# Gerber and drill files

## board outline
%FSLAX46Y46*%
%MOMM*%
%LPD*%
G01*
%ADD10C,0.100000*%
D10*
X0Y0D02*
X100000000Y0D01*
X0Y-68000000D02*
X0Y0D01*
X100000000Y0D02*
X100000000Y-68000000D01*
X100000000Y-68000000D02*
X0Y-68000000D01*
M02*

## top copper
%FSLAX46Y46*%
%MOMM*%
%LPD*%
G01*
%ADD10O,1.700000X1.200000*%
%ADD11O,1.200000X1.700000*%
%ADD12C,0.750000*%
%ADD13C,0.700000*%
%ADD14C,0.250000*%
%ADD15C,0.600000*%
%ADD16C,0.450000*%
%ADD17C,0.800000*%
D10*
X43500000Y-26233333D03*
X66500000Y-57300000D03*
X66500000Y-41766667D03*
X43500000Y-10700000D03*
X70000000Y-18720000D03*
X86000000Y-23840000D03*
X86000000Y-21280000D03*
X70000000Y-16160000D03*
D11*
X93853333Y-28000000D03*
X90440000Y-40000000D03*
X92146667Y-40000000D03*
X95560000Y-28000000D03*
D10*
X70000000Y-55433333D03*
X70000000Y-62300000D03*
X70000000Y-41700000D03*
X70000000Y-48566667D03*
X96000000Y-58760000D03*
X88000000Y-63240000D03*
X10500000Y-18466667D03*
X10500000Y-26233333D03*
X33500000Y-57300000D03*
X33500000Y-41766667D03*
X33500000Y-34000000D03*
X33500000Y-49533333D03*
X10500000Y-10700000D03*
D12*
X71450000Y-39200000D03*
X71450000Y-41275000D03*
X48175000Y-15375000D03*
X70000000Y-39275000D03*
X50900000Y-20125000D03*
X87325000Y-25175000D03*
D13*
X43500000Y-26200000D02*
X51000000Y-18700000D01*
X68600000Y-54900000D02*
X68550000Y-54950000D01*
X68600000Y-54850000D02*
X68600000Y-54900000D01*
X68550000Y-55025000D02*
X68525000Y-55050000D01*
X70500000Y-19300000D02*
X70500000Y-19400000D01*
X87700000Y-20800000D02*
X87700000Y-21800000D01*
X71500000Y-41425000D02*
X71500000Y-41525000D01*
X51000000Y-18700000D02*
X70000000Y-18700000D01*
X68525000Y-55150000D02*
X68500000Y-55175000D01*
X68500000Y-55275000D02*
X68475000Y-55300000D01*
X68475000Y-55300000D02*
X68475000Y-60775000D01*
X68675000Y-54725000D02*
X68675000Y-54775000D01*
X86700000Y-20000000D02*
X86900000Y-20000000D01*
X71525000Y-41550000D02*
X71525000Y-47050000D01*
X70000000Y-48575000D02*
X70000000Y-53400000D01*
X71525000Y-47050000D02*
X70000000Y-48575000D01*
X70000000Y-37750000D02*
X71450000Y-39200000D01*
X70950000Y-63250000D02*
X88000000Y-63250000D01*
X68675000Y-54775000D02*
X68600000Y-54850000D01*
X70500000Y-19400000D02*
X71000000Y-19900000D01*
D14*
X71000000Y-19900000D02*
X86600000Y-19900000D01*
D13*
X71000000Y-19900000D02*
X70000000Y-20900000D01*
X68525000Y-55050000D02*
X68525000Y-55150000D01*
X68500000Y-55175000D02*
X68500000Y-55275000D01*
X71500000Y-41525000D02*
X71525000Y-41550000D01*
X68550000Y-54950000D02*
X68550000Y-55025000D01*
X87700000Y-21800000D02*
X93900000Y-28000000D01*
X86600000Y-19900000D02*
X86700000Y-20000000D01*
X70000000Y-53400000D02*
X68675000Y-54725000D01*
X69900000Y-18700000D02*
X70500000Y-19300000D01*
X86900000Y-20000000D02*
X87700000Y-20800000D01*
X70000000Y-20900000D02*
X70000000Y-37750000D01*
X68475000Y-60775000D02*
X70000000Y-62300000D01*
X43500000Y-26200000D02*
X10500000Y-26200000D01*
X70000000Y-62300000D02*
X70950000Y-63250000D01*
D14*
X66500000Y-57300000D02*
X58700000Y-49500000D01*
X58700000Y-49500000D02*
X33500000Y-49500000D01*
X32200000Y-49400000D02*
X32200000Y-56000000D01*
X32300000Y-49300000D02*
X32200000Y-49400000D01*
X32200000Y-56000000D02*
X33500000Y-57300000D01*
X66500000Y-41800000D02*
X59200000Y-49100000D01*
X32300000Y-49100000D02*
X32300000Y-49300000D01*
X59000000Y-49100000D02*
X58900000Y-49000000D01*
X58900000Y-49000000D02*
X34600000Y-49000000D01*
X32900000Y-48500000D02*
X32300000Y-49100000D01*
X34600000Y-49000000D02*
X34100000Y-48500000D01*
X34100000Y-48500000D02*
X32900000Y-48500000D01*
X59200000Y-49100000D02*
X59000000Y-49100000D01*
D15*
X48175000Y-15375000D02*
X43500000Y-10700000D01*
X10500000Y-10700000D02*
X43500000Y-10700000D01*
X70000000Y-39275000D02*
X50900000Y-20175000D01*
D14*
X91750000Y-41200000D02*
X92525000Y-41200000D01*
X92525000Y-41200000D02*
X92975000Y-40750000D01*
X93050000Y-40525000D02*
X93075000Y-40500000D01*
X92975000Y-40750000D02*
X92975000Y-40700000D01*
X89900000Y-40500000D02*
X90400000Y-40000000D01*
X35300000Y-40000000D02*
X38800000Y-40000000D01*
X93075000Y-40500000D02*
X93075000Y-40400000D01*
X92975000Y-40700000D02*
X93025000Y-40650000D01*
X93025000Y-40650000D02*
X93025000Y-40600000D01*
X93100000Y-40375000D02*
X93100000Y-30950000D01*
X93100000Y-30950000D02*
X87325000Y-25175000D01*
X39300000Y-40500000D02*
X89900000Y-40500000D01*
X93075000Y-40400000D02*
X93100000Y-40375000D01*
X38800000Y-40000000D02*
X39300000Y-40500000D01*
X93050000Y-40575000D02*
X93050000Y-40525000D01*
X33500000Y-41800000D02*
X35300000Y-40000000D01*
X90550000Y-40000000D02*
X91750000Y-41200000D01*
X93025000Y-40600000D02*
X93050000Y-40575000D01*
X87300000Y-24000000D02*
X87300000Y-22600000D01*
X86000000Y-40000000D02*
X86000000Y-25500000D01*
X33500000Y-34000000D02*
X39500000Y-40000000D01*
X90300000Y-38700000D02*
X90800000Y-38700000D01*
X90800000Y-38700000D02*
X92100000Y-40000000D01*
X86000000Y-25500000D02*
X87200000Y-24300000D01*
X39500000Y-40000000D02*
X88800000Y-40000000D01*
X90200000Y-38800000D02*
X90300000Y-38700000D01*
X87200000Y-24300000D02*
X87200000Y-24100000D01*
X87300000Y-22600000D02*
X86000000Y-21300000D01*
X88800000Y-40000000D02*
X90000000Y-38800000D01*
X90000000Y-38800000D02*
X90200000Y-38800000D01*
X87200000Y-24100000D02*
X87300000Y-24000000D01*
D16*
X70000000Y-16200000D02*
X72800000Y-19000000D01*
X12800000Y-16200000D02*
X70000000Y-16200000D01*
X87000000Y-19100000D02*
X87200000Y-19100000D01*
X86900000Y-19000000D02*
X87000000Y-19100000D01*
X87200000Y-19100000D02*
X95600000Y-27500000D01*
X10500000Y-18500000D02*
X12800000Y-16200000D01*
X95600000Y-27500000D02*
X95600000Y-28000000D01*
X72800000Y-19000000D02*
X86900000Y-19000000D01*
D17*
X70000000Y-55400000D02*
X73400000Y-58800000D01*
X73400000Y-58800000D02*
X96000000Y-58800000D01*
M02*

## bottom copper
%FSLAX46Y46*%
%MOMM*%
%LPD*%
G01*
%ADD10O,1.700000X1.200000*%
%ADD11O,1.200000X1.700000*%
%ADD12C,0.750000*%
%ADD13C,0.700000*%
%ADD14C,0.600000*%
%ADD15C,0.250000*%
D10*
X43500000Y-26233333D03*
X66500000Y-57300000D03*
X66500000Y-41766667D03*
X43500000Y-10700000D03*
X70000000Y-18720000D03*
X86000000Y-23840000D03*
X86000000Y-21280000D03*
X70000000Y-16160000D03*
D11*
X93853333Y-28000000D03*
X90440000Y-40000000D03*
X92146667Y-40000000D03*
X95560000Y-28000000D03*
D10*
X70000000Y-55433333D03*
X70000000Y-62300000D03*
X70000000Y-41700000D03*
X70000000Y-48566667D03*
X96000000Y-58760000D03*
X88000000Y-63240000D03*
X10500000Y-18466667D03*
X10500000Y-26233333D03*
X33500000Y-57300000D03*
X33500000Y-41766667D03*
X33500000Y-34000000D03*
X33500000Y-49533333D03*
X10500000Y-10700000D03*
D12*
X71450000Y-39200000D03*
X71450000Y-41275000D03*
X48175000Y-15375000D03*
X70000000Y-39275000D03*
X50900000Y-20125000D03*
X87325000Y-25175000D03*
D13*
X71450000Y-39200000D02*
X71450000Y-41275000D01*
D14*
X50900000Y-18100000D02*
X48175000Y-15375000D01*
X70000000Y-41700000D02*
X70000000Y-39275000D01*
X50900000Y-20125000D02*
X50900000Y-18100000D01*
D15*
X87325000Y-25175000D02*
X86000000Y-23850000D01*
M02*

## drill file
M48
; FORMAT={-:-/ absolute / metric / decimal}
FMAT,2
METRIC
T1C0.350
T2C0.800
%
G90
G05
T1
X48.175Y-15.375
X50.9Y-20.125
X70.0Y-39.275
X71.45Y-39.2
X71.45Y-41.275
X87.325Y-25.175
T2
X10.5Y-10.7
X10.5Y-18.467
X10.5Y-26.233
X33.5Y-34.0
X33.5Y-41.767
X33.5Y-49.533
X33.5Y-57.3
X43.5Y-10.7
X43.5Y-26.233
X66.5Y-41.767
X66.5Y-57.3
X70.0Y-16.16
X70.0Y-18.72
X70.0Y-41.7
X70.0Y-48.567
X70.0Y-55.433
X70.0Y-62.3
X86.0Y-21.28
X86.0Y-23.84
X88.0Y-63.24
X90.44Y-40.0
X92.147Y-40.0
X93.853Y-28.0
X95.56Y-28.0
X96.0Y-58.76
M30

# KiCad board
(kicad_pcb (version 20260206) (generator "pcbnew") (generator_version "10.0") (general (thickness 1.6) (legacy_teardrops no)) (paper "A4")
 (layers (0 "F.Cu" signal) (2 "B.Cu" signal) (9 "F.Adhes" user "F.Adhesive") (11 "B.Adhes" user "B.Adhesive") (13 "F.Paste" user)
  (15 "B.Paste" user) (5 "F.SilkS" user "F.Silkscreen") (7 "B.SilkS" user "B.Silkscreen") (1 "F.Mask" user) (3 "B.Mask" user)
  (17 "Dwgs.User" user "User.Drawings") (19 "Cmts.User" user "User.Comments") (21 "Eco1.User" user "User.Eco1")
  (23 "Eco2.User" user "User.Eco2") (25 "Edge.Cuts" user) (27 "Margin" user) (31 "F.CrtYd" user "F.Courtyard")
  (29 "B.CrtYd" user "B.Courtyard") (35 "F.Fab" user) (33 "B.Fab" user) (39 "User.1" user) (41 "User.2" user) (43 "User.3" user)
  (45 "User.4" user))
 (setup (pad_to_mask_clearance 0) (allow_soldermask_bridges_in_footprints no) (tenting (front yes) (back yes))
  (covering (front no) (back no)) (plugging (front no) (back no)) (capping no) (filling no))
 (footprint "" (layer "F.Cu") (at 55 34)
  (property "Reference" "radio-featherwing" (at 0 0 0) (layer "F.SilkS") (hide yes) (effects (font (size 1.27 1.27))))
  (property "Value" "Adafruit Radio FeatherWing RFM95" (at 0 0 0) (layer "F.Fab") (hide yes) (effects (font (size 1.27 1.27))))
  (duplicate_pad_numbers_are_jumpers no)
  (pad "GND" thru_hole oval (at -11.5 -7.766667) (size 1.7 1.2) (drill 0.8) (layers "*.Cu") (remove_unused_layers no) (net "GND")
   (thermal_bridge_angle 45))
  (pad "RX" thru_hole oval (at 11.5 23.3) (size 1.7 1.2) (drill 0.8) (layers "*.Cu") (remove_unused_layers no) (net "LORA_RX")
   (thermal_bridge_angle 45))
  (pad "TX" thru_hole oval (at 11.5 7.766667) (size 1.7 1.2) (drill 0.8) (layers "*.Cu") (remove_unused_layers no) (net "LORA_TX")
   (thermal_bridge_angle 45))
  (pad "VCC" thru_hole oval (at -11.5 -23.3) (size 1.7 1.2) (drill 0.8) (layers "*.Cu") (remove_unused_layers no) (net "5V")
   (thermal_bridge_angle 45)))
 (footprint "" (layer "F.Cu") (at 78 20)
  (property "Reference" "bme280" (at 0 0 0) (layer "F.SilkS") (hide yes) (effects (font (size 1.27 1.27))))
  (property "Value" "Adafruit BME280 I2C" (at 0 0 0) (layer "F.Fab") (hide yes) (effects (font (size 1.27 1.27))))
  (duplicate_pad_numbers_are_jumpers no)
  (pad "GND" thru_hole oval (at -8 -1.28) (size 1.7 1.2) (drill 0.8) (layers "*.Cu") (remove_unused_layers no) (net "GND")
   (thermal_bridge_angle 45))
  (pad "SCL" thru_hole oval (at 8 3.84) (size 1.7 1.2) (drill 0.8) (layers "*.Cu") (remove_unused_layers no) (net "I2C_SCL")
   (thermal_bridge_angle 45))
  (pad "SDA" thru_hole oval (at 8 1.28) (size 1.7 1.2) (drill 0.8) (layers "*.Cu") (remove_unused_layers no) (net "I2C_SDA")
   (thermal_bridge_angle 45))
  (pad "VCC" thru_hole oval (at -8 -3.84) (size 1.7 1.2) (drill 0.8) (layers "*.Cu") (remove_unused_layers no) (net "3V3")
   (thermal_bridge_angle 45)))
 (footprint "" (layer "F.Cu") (at 93 34 90)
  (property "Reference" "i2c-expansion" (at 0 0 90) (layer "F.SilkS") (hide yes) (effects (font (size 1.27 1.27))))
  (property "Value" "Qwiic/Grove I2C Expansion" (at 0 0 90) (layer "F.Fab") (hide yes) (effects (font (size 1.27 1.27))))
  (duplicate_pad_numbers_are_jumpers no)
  (pad "GND" thru_hole oval (at 6 0.853333 90) (size 1.7 1.2) (drill 0.8) (layers "*.Cu") (remove_unused_layers no) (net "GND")
   (thermal_bridge_angle 45))
  (pad "SCL" thru_hole oval (at -6 -2.56 90) (size 1.7 1.2) (drill 0.8) (layers "*.Cu") (remove_unused_layers no) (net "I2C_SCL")
   (thermal_bridge_angle 45))
  (pad "SDA" thru_hole oval (at -6 -0.853333 90) (size 1.7 1.2) (drill 0.8) (layers "*.Cu") (remove_unused_layers no) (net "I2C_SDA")
   (thermal_bridge_angle 45))
  (pad "VCC" thru_hole oval (at 6 2.56 90) (size 1.7 1.2) (drill 0.8) (layers "*.Cu") (remove_unused_layers no) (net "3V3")
   (thermal_bridge_angle 45)))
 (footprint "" (layer "F.Cu") (at 78 52)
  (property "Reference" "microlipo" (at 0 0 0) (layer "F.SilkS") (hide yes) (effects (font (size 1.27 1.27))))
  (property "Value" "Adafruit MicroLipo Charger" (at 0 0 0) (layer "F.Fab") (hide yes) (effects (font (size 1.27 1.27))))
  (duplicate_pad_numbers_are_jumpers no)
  (pad "B+" thru_hole oval (at -8 3.433333) (size 1.7 1.2) (drill 0.8) (layers "*.Cu") (remove_unused_layers no) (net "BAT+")
   (thermal_bridge_angle 45))
  (pad "B-" thru_hole oval (at -8 10.3) (size 1.7 1.2) (drill 0.8) (layers "*.Cu") (remove_unused_layers no) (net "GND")
   (thermal_bridge_angle 45))
  (pad "OUT+" thru_hole oval (at -8 -10.3) (size 1.7 1.2) (drill 0.8) (layers "*.Cu") (remove_unused_layers no) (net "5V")
   (thermal_bridge_angle 45))
  (pad "OUT-" thru_hole oval (at -8 -3.433333) (size 1.7 1.2) (drill 0.8) (layers "*.Cu") (remove_unused_layers no) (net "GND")
   (thermal_bridge_angle 45)))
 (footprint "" (layer "F.Cu") (at 92 61)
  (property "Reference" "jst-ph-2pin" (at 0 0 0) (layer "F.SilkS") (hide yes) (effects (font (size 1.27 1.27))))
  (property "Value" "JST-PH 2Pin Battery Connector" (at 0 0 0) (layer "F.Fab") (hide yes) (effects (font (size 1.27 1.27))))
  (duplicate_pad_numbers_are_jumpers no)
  (pad "BAT+" thru_hole oval (at 4 -2.24) (size 1.7 1.2) (drill 0.8) (layers "*.Cu") (remove_unused_layers no) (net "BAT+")
   (thermal_bridge_angle 45))
  (pad "GND" thru_hole oval (at -4 2.24) (size 1.7 1.2) (drill 0.8) (layers "*.Cu") (remove_unused_layers no) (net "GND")
   (thermal_bridge_angle 45)))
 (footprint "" (layer "F.Cu") (at 22 34)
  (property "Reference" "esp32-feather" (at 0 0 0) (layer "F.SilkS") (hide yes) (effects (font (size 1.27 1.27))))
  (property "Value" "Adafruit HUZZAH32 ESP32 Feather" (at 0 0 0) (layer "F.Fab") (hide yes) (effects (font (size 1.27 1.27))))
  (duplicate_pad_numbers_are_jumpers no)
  (pad "3V3" thru_hole oval (at -11.5 -15.533333) (size 1.7 1.2) (drill 0.8) (layers "*.Cu") (remove_unused_layers no) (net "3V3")
   (thermal_bridge_angle 45))
  (pad "GND" thru_hole oval (at -11.5 -7.766667) (size 1.7 1.2) (drill 0.8) (layers "*.Cu") (remove_unused_layers no) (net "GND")
   (thermal_bridge_angle 45))
  (pad "RX" thru_hole oval (at 11.5 23.3) (size 1.7 1.2) (drill 0.8) (layers "*.Cu") (remove_unused_layers no) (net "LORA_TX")
   (thermal_bridge_angle 45))
  (pad "SCL" thru_hole oval (at 11.5 7.766667) (size 1.7 1.2) (drill 0.8) (layers "*.Cu") (remove_unused_layers no) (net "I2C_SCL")
   (thermal_bridge_angle 45))
  (pad "SDA" thru_hole oval (at 11.5 0) (size 1.7 1.2) (drill 0.8) (layers "*.Cu") (remove_unused_layers no) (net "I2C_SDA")
   (thermal_bridge_angle 45))
  (pad "TX" thru_hole oval (at 11.5 15.533333) (size 1.7 1.2) (drill 0.8) (layers "*.Cu") (remove_unused_layers no) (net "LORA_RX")
   (thermal_bridge_angle 45))
  (pad "VIN" thru_hole oval (at -11.5 -23.3) (size 1.7 1.2) (drill 0.8) (layers "*.Cu") (remove_unused_layers no) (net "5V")
   (thermal_bridge_angle 45)))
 (gr_line (start 0 0) (end 100 0) (stroke (width 0.1) (type default)) (layer "Edge.Cuts"))
 (gr_line (start 0 68) (end 0 0) (stroke (width 0.1) (type default)) (layer "Edge.Cuts"))
 (gr_line (start 100 0) (end 100 68) (stroke (width 0.1) (type default)) (layer "Edge.Cuts"))
 (gr_line (start 100 68) (end 0 68) (stroke (width 0.1) (type default)) (layer "Edge.Cuts"))
 (segment (start 43.5 26.2) (end 51 18.7) (width 0.7) (layer "F.Cu") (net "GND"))
 (segment (start 68.6 54.9) (end 68.55 54.95) (width 0.7) (layer "F.Cu") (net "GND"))
 (segment (start 68.6 54.85) (end 68.6 54.9) (width 0.7) (layer "F.Cu") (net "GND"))
 (segment (start 68.55 55.025) (end 68.525 55.05) (width 0.7) (layer "F.Cu") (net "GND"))
 (segment (start 70.5 19.3) (end 70.5 19.4) (width 0.7) (layer "F.Cu") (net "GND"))
 (segment (start 87.7 20.8) (end 87.7 21.8) (width 0.7) (layer "F.Cu") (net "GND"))
 (segment (start 71.5 41.425) (end 71.5 41.525) (width 0.7) (layer "F.Cu") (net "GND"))
 (segment (start 51 18.7) (end 70 18.7) (width 0.7) (layer "F.Cu") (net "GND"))
 (segment (start 68.525 55.15) (end 68.5 55.175) (width 0.7) (layer "F.Cu") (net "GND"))
 (segment (start 68.5 55.275) (end 68.475 55.3) (width 0.7) (layer "F.Cu") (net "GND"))
 (segment (start 68.475 55.3) (end 68.475 60.775) (width 0.7) (layer "F.Cu") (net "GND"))
 (segment (start 68.675 54.725) (end 68.675 54.775) (width 0.7) (layer "F.Cu") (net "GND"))
 (segment (start 86.7 20) (end 86.9 20) (width 0.7) (layer "F.Cu") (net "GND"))
 (segment (start 71.525 41.55) (end 71.525 47.05) (width 0.7) (layer "F.Cu") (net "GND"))
 (segment (start 70 48.575) (end 70 53.4) (width 0.7) (layer "F.Cu") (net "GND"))
 (segment (start 71.525 47.05) (end 70 48.575) (width 0.7) (layer "F.Cu") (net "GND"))
 (segment (start 70 37.75) (end 71.45 39.2) (width 0.7) (layer "F.Cu") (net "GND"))
 (segment (start 70.95 63.25) (end 88 63.25) (width 0.7) (layer "F.Cu") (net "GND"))
 (segment (start 68.675 54.775) (end 68.6 54.85) (width 0.7) (layer "F.Cu") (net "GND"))
 (segment (start 70.5 19.4) (end 71 19.9) (width 0.7) (layer "F.Cu") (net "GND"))
 (segment (start 71 19.9) (end 86.6 19.9) (width 0.25) (layer "F.Cu") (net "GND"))
 (segment (start 71 19.9) (end 70 20.9) (width 0.7) (layer "F.Cu") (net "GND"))
 (segment (start 68.525 55.05) (end 68.525 55.15) (width 0.7) (layer "F.Cu") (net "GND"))
 (segment (start 68.5 55.175) (end 68.5 55.275) (width 0.7) (layer "F.Cu") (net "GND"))
 (segment (start 71.5 41.525) (end 71.525 41.55) (width 0.7) (layer "F.Cu") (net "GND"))
 (segment (start 68.55 54.95) (end 68.55 55.025) (width 0.7) (layer "F.Cu") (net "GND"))
 (segment (start 87.7 21.8) (end 93.9 28) (width 0.7) (layer "F.Cu") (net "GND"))
 (segment (start 86.6 19.9) (end 86.7 20) (width 0.7) (layer "F.Cu") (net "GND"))
 (segment (start 70 53.4) (end 68.675 54.725) (width 0.7) (layer "F.Cu") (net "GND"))
 (segment (start 69.9 18.7) (end 70.5 19.3) (width 0.7) (layer "F.Cu") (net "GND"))
 (segment (start 86.9 20) (end 87.7 20.8) (width 0.7) (layer "F.Cu") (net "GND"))
 (segment (start 70 20.9) (end 70 37.75) (width 0.7) (layer "F.Cu") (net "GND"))
 (segment (start 68.475 60.775) (end 70 62.3) (width 0.7) (layer "F.Cu") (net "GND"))
 (segment (start 43.5 26.2) (end 10.5 26.2) (width 0.7) (layer "F.Cu") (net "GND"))
 (segment (start 70 62.3) (end 70.95 63.25) (width 0.7) (layer "F.Cu") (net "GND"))
 (via (at 71.45 39.2) (size 0.75) (drill 0.35) (layers "F.Cu" "B.Cu") (tenting (front yes) (back yes)) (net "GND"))
 (via (at 71.45 41.275) (size 0.75) (drill 0.35) (layers "F.Cu" "B.Cu") (tenting (front yes) (back yes)) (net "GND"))
 (segment (start 71.45 39.2) (end 71.45 41.275) (width 0.7) (layer "B.Cu") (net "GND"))
 (segment (start 66.5 57.3) (end 58.7 49.5) (width 0.25) (layer "F.Cu") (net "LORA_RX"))
 (segment (start 58.7 49.5) (end 33.5 49.5) (width 0.25) (layer "F.Cu") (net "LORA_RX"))
 (segment (start 32.2 49.4) (end 32.2 56) (width 0.25) (layer "F.Cu") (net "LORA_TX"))
 (segment (start 32.3 49.3) (end 32.2 49.4) (width 0.25) (layer "F.Cu") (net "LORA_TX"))
 (segment (start 32.2 56) (end 33.5 57.3) (width 0.25) (layer "F.Cu") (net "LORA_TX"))
 (segment (start 66.5 41.8) (end 59.2 49.1) (width 0.25) (layer "F.Cu") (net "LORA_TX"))
 (segment (start 32.3 49.1) (end 32.3 49.3) (width 0.25) (layer "F.Cu") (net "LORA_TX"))
 (segment (start 59 49.1) (end 58.9 49) (width 0.25) (layer "F.Cu") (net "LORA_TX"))
 (segment (start 58.9 49) (end 34.6 49) (width 0.25) (layer "F.Cu") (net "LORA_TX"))
 (segment (start 32.9 48.5) (end 32.3 49.1) (width 0.25) (layer "F.Cu") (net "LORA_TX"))
 (segment (start 34.6 49) (end 34.1 48.5) (width 0.25) (layer "F.Cu") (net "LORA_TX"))
 (segment (start 34.1 48.5) (end 32.9 48.5) (width 0.25) (layer "F.Cu") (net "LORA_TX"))
 (segment (start 59.2 49.1) (end 59 49.1) (width 0.25) (layer "F.Cu") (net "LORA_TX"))
 (segment (start 48.175 15.375) (end 43.5 10.7) (width 0.6) (layer "F.Cu") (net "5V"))
 (segment (start 10.5 10.7) (end 43.5 10.7) (width 0.6) (layer "F.Cu") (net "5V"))
 (segment (start 70 39.275) (end 50.9 20.175) (width 0.6) (layer "F.Cu") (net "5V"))
 (via (at 48.175 15.375) (size 0.75) (drill 0.35) (layers "F.Cu" "B.Cu") (tenting (front yes) (back yes)) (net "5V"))
 (via (at 70 39.275) (size 0.75) (drill 0.35) (layers "F.Cu" "B.Cu") (tenting (front yes) (back yes)) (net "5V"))
 (via (at 50.9 20.125) (size 0.75) (drill 0.35) (layers "F.Cu" "B.Cu") (tenting (front yes) (back yes)) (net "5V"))
 (segment (start 50.9 18.1) (end 48.175 15.375) (width 0.6) (layer "B.Cu") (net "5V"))
 (segment (start 70 41.7) (end 70 39.275) (width 0.6) (layer "B.Cu") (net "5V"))
 (segment (start 50.9 20.125) (end 50.9 18.1) (width 0.6) (layer "B.Cu") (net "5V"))
 (segment (start 91.75 41.2) (end 92.525 41.2) (width 0.25) (layer "F.Cu") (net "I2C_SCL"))
 (segment (start 92.525 41.2) (end 92.975 40.75) (width 0.25) (layer "F.Cu") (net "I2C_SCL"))
 (segment (start 93.05 40.525) (end 93.075 40.5) (width 0.25) (layer "F.Cu") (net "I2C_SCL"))
 (segment (start 92.975 40.75) (end 92.975 40.7) (width 0.25) (layer "F.Cu") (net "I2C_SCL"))
 (segment (start 89.9 40.5) (end 90.4 40) (width 0.25) (layer "F.Cu") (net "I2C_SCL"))
 (segment (start 35.3 40) (end 38.8 40) (width 0.25) (layer "F.Cu") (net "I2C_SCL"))
 (segment (start 93.075 40.5) (end 93.075 40.4) (width 0.25) (layer "F.Cu") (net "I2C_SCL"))
 (segment (start 92.975 40.7) (end 93.025 40.65) (width 0.25) (layer "F.Cu") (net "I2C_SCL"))
 (segment (start 93.025 40.65) (end 93.025 40.6) (width 0.25) (layer "F.Cu") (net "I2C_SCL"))
 (segment (start 93.1 40.375) (end 93.1 30.95) (width 0.25) (layer "F.Cu") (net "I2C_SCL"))
 (segment (start 93.1 30.95) (end 87.325 25.175) (width 0.25) (layer "F.Cu") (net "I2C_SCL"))
 (segment (start 39.3 40.5) (end 89.9 40.5) (width 0.25) (layer "F.Cu") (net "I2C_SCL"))
 (segment (start 93.075 40.4) (end 93.1 40.375) (width 0.25) (layer "F.Cu") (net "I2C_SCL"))
 (segment (start 38.8 40) (end 39.3 40.5) (width 0.25) (layer "F.Cu") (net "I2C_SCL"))
 (segment (start 93.05 40.575) (end 93.05 40.525) (width 0.25) (layer "F.Cu") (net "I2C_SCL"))
 (segment (start 33.5 41.8) (end 35.3 40) (width 0.25) (layer "F.Cu") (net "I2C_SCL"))
 (segment (start 90.55 40) (end 91.75 41.2) (width 0.25) (layer "F.Cu") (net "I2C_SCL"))
 (segment (start 93.025 40.6) (end 93.05 40.575) (width 0.25) (layer "F.Cu") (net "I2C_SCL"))
 (via (at 87.325 25.175) (size 0.75) (drill 0.35) (layers "F.Cu" "B.Cu") (tenting (front yes) (back yes)) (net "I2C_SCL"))
 (segment (start 87.325 25.175) (end 86 23.85) (width 0.25) (layer "B.Cu") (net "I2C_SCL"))
 (segment (start 87.3 24) (end 87.3 22.6) (width 0.25) (layer "F.Cu") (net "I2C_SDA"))
 (segment (start 86 40) (end 86 25.5) (width 0.25) (layer "F.Cu") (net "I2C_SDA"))
 (segment (start 33.5 34) (end 39.5 40) (width 0.25) (layer "F.Cu") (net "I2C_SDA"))
 (segment (start 90.3 38.7) (end 90.8 38.7) (width 0.25) (layer "F.Cu") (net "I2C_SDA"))
 (segment (start 90.8 38.7) (end 92.1 40) (width 0.25) (layer "F.Cu") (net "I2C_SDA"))
 (segment (start 86 25.5) (end 87.2 24.3) (width 0.25) (layer "F.Cu") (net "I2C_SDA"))
 (segment (start 39.5 40) (end 88.8 40) (width 0.25) (layer "F.Cu") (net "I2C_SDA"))
 (segment (start 90.2 38.8) (end 90.3 38.7) (width 0.25) (layer "F.Cu") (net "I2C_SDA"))
 (segment (start 87.2 24.3) (end 87.2 24.1) (width 0.25) (layer "F.Cu") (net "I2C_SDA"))
 (segment (start 87.3 22.6) (end 86 21.3) (width 0.25) (layer "F.Cu") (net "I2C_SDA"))
 (segment (start 88.8 40) (end 90 38.8) (width 0.25) (layer "F.Cu") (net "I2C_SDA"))
 (segment (start 90 38.8) (end 90.2 38.8) (width 0.25) (layer "F.Cu") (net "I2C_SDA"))
 (segment (start 87.2 24.1) (end 87.3 24) (width 0.25) (layer "F.Cu") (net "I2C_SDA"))
 (segment (start 70 16.2) (end 72.8 19) (width 0.45) (layer "F.Cu") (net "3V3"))
 (segment (start 12.8 16.2) (end 70 16.2) (width 0.45) (layer "F.Cu") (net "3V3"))
 (segment (start 87 19.1) (end 87.2 19.1) (width 0.45) (layer "F.Cu") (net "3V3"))
 (segment (start 86.9 19) (end 87 19.1) (width 0.45) (layer "F.Cu") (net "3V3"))
 (segment (start 87.2 19.1) (end 95.6 27.5) (width 0.45) (layer "F.Cu") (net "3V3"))
 (segment (start 10.5 18.5) (end 12.8 16.2) (width 0.45) (layer "F.Cu") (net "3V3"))
 (segment (start 95.6 27.5) (end 95.6 28) (width 0.45) (layer "F.Cu") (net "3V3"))
 (segment (start 72.8 19) (end 86.9 19) (width 0.45) (layer "F.Cu") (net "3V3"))
 (segment (start 70 55.4) (end 73.4 58.8) (width 0.8) (layer "F.Cu") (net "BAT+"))
 (segment (start 73.4 58.8) (end 96 58.8) (width 0.8) (layer "F.Cu") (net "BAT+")))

